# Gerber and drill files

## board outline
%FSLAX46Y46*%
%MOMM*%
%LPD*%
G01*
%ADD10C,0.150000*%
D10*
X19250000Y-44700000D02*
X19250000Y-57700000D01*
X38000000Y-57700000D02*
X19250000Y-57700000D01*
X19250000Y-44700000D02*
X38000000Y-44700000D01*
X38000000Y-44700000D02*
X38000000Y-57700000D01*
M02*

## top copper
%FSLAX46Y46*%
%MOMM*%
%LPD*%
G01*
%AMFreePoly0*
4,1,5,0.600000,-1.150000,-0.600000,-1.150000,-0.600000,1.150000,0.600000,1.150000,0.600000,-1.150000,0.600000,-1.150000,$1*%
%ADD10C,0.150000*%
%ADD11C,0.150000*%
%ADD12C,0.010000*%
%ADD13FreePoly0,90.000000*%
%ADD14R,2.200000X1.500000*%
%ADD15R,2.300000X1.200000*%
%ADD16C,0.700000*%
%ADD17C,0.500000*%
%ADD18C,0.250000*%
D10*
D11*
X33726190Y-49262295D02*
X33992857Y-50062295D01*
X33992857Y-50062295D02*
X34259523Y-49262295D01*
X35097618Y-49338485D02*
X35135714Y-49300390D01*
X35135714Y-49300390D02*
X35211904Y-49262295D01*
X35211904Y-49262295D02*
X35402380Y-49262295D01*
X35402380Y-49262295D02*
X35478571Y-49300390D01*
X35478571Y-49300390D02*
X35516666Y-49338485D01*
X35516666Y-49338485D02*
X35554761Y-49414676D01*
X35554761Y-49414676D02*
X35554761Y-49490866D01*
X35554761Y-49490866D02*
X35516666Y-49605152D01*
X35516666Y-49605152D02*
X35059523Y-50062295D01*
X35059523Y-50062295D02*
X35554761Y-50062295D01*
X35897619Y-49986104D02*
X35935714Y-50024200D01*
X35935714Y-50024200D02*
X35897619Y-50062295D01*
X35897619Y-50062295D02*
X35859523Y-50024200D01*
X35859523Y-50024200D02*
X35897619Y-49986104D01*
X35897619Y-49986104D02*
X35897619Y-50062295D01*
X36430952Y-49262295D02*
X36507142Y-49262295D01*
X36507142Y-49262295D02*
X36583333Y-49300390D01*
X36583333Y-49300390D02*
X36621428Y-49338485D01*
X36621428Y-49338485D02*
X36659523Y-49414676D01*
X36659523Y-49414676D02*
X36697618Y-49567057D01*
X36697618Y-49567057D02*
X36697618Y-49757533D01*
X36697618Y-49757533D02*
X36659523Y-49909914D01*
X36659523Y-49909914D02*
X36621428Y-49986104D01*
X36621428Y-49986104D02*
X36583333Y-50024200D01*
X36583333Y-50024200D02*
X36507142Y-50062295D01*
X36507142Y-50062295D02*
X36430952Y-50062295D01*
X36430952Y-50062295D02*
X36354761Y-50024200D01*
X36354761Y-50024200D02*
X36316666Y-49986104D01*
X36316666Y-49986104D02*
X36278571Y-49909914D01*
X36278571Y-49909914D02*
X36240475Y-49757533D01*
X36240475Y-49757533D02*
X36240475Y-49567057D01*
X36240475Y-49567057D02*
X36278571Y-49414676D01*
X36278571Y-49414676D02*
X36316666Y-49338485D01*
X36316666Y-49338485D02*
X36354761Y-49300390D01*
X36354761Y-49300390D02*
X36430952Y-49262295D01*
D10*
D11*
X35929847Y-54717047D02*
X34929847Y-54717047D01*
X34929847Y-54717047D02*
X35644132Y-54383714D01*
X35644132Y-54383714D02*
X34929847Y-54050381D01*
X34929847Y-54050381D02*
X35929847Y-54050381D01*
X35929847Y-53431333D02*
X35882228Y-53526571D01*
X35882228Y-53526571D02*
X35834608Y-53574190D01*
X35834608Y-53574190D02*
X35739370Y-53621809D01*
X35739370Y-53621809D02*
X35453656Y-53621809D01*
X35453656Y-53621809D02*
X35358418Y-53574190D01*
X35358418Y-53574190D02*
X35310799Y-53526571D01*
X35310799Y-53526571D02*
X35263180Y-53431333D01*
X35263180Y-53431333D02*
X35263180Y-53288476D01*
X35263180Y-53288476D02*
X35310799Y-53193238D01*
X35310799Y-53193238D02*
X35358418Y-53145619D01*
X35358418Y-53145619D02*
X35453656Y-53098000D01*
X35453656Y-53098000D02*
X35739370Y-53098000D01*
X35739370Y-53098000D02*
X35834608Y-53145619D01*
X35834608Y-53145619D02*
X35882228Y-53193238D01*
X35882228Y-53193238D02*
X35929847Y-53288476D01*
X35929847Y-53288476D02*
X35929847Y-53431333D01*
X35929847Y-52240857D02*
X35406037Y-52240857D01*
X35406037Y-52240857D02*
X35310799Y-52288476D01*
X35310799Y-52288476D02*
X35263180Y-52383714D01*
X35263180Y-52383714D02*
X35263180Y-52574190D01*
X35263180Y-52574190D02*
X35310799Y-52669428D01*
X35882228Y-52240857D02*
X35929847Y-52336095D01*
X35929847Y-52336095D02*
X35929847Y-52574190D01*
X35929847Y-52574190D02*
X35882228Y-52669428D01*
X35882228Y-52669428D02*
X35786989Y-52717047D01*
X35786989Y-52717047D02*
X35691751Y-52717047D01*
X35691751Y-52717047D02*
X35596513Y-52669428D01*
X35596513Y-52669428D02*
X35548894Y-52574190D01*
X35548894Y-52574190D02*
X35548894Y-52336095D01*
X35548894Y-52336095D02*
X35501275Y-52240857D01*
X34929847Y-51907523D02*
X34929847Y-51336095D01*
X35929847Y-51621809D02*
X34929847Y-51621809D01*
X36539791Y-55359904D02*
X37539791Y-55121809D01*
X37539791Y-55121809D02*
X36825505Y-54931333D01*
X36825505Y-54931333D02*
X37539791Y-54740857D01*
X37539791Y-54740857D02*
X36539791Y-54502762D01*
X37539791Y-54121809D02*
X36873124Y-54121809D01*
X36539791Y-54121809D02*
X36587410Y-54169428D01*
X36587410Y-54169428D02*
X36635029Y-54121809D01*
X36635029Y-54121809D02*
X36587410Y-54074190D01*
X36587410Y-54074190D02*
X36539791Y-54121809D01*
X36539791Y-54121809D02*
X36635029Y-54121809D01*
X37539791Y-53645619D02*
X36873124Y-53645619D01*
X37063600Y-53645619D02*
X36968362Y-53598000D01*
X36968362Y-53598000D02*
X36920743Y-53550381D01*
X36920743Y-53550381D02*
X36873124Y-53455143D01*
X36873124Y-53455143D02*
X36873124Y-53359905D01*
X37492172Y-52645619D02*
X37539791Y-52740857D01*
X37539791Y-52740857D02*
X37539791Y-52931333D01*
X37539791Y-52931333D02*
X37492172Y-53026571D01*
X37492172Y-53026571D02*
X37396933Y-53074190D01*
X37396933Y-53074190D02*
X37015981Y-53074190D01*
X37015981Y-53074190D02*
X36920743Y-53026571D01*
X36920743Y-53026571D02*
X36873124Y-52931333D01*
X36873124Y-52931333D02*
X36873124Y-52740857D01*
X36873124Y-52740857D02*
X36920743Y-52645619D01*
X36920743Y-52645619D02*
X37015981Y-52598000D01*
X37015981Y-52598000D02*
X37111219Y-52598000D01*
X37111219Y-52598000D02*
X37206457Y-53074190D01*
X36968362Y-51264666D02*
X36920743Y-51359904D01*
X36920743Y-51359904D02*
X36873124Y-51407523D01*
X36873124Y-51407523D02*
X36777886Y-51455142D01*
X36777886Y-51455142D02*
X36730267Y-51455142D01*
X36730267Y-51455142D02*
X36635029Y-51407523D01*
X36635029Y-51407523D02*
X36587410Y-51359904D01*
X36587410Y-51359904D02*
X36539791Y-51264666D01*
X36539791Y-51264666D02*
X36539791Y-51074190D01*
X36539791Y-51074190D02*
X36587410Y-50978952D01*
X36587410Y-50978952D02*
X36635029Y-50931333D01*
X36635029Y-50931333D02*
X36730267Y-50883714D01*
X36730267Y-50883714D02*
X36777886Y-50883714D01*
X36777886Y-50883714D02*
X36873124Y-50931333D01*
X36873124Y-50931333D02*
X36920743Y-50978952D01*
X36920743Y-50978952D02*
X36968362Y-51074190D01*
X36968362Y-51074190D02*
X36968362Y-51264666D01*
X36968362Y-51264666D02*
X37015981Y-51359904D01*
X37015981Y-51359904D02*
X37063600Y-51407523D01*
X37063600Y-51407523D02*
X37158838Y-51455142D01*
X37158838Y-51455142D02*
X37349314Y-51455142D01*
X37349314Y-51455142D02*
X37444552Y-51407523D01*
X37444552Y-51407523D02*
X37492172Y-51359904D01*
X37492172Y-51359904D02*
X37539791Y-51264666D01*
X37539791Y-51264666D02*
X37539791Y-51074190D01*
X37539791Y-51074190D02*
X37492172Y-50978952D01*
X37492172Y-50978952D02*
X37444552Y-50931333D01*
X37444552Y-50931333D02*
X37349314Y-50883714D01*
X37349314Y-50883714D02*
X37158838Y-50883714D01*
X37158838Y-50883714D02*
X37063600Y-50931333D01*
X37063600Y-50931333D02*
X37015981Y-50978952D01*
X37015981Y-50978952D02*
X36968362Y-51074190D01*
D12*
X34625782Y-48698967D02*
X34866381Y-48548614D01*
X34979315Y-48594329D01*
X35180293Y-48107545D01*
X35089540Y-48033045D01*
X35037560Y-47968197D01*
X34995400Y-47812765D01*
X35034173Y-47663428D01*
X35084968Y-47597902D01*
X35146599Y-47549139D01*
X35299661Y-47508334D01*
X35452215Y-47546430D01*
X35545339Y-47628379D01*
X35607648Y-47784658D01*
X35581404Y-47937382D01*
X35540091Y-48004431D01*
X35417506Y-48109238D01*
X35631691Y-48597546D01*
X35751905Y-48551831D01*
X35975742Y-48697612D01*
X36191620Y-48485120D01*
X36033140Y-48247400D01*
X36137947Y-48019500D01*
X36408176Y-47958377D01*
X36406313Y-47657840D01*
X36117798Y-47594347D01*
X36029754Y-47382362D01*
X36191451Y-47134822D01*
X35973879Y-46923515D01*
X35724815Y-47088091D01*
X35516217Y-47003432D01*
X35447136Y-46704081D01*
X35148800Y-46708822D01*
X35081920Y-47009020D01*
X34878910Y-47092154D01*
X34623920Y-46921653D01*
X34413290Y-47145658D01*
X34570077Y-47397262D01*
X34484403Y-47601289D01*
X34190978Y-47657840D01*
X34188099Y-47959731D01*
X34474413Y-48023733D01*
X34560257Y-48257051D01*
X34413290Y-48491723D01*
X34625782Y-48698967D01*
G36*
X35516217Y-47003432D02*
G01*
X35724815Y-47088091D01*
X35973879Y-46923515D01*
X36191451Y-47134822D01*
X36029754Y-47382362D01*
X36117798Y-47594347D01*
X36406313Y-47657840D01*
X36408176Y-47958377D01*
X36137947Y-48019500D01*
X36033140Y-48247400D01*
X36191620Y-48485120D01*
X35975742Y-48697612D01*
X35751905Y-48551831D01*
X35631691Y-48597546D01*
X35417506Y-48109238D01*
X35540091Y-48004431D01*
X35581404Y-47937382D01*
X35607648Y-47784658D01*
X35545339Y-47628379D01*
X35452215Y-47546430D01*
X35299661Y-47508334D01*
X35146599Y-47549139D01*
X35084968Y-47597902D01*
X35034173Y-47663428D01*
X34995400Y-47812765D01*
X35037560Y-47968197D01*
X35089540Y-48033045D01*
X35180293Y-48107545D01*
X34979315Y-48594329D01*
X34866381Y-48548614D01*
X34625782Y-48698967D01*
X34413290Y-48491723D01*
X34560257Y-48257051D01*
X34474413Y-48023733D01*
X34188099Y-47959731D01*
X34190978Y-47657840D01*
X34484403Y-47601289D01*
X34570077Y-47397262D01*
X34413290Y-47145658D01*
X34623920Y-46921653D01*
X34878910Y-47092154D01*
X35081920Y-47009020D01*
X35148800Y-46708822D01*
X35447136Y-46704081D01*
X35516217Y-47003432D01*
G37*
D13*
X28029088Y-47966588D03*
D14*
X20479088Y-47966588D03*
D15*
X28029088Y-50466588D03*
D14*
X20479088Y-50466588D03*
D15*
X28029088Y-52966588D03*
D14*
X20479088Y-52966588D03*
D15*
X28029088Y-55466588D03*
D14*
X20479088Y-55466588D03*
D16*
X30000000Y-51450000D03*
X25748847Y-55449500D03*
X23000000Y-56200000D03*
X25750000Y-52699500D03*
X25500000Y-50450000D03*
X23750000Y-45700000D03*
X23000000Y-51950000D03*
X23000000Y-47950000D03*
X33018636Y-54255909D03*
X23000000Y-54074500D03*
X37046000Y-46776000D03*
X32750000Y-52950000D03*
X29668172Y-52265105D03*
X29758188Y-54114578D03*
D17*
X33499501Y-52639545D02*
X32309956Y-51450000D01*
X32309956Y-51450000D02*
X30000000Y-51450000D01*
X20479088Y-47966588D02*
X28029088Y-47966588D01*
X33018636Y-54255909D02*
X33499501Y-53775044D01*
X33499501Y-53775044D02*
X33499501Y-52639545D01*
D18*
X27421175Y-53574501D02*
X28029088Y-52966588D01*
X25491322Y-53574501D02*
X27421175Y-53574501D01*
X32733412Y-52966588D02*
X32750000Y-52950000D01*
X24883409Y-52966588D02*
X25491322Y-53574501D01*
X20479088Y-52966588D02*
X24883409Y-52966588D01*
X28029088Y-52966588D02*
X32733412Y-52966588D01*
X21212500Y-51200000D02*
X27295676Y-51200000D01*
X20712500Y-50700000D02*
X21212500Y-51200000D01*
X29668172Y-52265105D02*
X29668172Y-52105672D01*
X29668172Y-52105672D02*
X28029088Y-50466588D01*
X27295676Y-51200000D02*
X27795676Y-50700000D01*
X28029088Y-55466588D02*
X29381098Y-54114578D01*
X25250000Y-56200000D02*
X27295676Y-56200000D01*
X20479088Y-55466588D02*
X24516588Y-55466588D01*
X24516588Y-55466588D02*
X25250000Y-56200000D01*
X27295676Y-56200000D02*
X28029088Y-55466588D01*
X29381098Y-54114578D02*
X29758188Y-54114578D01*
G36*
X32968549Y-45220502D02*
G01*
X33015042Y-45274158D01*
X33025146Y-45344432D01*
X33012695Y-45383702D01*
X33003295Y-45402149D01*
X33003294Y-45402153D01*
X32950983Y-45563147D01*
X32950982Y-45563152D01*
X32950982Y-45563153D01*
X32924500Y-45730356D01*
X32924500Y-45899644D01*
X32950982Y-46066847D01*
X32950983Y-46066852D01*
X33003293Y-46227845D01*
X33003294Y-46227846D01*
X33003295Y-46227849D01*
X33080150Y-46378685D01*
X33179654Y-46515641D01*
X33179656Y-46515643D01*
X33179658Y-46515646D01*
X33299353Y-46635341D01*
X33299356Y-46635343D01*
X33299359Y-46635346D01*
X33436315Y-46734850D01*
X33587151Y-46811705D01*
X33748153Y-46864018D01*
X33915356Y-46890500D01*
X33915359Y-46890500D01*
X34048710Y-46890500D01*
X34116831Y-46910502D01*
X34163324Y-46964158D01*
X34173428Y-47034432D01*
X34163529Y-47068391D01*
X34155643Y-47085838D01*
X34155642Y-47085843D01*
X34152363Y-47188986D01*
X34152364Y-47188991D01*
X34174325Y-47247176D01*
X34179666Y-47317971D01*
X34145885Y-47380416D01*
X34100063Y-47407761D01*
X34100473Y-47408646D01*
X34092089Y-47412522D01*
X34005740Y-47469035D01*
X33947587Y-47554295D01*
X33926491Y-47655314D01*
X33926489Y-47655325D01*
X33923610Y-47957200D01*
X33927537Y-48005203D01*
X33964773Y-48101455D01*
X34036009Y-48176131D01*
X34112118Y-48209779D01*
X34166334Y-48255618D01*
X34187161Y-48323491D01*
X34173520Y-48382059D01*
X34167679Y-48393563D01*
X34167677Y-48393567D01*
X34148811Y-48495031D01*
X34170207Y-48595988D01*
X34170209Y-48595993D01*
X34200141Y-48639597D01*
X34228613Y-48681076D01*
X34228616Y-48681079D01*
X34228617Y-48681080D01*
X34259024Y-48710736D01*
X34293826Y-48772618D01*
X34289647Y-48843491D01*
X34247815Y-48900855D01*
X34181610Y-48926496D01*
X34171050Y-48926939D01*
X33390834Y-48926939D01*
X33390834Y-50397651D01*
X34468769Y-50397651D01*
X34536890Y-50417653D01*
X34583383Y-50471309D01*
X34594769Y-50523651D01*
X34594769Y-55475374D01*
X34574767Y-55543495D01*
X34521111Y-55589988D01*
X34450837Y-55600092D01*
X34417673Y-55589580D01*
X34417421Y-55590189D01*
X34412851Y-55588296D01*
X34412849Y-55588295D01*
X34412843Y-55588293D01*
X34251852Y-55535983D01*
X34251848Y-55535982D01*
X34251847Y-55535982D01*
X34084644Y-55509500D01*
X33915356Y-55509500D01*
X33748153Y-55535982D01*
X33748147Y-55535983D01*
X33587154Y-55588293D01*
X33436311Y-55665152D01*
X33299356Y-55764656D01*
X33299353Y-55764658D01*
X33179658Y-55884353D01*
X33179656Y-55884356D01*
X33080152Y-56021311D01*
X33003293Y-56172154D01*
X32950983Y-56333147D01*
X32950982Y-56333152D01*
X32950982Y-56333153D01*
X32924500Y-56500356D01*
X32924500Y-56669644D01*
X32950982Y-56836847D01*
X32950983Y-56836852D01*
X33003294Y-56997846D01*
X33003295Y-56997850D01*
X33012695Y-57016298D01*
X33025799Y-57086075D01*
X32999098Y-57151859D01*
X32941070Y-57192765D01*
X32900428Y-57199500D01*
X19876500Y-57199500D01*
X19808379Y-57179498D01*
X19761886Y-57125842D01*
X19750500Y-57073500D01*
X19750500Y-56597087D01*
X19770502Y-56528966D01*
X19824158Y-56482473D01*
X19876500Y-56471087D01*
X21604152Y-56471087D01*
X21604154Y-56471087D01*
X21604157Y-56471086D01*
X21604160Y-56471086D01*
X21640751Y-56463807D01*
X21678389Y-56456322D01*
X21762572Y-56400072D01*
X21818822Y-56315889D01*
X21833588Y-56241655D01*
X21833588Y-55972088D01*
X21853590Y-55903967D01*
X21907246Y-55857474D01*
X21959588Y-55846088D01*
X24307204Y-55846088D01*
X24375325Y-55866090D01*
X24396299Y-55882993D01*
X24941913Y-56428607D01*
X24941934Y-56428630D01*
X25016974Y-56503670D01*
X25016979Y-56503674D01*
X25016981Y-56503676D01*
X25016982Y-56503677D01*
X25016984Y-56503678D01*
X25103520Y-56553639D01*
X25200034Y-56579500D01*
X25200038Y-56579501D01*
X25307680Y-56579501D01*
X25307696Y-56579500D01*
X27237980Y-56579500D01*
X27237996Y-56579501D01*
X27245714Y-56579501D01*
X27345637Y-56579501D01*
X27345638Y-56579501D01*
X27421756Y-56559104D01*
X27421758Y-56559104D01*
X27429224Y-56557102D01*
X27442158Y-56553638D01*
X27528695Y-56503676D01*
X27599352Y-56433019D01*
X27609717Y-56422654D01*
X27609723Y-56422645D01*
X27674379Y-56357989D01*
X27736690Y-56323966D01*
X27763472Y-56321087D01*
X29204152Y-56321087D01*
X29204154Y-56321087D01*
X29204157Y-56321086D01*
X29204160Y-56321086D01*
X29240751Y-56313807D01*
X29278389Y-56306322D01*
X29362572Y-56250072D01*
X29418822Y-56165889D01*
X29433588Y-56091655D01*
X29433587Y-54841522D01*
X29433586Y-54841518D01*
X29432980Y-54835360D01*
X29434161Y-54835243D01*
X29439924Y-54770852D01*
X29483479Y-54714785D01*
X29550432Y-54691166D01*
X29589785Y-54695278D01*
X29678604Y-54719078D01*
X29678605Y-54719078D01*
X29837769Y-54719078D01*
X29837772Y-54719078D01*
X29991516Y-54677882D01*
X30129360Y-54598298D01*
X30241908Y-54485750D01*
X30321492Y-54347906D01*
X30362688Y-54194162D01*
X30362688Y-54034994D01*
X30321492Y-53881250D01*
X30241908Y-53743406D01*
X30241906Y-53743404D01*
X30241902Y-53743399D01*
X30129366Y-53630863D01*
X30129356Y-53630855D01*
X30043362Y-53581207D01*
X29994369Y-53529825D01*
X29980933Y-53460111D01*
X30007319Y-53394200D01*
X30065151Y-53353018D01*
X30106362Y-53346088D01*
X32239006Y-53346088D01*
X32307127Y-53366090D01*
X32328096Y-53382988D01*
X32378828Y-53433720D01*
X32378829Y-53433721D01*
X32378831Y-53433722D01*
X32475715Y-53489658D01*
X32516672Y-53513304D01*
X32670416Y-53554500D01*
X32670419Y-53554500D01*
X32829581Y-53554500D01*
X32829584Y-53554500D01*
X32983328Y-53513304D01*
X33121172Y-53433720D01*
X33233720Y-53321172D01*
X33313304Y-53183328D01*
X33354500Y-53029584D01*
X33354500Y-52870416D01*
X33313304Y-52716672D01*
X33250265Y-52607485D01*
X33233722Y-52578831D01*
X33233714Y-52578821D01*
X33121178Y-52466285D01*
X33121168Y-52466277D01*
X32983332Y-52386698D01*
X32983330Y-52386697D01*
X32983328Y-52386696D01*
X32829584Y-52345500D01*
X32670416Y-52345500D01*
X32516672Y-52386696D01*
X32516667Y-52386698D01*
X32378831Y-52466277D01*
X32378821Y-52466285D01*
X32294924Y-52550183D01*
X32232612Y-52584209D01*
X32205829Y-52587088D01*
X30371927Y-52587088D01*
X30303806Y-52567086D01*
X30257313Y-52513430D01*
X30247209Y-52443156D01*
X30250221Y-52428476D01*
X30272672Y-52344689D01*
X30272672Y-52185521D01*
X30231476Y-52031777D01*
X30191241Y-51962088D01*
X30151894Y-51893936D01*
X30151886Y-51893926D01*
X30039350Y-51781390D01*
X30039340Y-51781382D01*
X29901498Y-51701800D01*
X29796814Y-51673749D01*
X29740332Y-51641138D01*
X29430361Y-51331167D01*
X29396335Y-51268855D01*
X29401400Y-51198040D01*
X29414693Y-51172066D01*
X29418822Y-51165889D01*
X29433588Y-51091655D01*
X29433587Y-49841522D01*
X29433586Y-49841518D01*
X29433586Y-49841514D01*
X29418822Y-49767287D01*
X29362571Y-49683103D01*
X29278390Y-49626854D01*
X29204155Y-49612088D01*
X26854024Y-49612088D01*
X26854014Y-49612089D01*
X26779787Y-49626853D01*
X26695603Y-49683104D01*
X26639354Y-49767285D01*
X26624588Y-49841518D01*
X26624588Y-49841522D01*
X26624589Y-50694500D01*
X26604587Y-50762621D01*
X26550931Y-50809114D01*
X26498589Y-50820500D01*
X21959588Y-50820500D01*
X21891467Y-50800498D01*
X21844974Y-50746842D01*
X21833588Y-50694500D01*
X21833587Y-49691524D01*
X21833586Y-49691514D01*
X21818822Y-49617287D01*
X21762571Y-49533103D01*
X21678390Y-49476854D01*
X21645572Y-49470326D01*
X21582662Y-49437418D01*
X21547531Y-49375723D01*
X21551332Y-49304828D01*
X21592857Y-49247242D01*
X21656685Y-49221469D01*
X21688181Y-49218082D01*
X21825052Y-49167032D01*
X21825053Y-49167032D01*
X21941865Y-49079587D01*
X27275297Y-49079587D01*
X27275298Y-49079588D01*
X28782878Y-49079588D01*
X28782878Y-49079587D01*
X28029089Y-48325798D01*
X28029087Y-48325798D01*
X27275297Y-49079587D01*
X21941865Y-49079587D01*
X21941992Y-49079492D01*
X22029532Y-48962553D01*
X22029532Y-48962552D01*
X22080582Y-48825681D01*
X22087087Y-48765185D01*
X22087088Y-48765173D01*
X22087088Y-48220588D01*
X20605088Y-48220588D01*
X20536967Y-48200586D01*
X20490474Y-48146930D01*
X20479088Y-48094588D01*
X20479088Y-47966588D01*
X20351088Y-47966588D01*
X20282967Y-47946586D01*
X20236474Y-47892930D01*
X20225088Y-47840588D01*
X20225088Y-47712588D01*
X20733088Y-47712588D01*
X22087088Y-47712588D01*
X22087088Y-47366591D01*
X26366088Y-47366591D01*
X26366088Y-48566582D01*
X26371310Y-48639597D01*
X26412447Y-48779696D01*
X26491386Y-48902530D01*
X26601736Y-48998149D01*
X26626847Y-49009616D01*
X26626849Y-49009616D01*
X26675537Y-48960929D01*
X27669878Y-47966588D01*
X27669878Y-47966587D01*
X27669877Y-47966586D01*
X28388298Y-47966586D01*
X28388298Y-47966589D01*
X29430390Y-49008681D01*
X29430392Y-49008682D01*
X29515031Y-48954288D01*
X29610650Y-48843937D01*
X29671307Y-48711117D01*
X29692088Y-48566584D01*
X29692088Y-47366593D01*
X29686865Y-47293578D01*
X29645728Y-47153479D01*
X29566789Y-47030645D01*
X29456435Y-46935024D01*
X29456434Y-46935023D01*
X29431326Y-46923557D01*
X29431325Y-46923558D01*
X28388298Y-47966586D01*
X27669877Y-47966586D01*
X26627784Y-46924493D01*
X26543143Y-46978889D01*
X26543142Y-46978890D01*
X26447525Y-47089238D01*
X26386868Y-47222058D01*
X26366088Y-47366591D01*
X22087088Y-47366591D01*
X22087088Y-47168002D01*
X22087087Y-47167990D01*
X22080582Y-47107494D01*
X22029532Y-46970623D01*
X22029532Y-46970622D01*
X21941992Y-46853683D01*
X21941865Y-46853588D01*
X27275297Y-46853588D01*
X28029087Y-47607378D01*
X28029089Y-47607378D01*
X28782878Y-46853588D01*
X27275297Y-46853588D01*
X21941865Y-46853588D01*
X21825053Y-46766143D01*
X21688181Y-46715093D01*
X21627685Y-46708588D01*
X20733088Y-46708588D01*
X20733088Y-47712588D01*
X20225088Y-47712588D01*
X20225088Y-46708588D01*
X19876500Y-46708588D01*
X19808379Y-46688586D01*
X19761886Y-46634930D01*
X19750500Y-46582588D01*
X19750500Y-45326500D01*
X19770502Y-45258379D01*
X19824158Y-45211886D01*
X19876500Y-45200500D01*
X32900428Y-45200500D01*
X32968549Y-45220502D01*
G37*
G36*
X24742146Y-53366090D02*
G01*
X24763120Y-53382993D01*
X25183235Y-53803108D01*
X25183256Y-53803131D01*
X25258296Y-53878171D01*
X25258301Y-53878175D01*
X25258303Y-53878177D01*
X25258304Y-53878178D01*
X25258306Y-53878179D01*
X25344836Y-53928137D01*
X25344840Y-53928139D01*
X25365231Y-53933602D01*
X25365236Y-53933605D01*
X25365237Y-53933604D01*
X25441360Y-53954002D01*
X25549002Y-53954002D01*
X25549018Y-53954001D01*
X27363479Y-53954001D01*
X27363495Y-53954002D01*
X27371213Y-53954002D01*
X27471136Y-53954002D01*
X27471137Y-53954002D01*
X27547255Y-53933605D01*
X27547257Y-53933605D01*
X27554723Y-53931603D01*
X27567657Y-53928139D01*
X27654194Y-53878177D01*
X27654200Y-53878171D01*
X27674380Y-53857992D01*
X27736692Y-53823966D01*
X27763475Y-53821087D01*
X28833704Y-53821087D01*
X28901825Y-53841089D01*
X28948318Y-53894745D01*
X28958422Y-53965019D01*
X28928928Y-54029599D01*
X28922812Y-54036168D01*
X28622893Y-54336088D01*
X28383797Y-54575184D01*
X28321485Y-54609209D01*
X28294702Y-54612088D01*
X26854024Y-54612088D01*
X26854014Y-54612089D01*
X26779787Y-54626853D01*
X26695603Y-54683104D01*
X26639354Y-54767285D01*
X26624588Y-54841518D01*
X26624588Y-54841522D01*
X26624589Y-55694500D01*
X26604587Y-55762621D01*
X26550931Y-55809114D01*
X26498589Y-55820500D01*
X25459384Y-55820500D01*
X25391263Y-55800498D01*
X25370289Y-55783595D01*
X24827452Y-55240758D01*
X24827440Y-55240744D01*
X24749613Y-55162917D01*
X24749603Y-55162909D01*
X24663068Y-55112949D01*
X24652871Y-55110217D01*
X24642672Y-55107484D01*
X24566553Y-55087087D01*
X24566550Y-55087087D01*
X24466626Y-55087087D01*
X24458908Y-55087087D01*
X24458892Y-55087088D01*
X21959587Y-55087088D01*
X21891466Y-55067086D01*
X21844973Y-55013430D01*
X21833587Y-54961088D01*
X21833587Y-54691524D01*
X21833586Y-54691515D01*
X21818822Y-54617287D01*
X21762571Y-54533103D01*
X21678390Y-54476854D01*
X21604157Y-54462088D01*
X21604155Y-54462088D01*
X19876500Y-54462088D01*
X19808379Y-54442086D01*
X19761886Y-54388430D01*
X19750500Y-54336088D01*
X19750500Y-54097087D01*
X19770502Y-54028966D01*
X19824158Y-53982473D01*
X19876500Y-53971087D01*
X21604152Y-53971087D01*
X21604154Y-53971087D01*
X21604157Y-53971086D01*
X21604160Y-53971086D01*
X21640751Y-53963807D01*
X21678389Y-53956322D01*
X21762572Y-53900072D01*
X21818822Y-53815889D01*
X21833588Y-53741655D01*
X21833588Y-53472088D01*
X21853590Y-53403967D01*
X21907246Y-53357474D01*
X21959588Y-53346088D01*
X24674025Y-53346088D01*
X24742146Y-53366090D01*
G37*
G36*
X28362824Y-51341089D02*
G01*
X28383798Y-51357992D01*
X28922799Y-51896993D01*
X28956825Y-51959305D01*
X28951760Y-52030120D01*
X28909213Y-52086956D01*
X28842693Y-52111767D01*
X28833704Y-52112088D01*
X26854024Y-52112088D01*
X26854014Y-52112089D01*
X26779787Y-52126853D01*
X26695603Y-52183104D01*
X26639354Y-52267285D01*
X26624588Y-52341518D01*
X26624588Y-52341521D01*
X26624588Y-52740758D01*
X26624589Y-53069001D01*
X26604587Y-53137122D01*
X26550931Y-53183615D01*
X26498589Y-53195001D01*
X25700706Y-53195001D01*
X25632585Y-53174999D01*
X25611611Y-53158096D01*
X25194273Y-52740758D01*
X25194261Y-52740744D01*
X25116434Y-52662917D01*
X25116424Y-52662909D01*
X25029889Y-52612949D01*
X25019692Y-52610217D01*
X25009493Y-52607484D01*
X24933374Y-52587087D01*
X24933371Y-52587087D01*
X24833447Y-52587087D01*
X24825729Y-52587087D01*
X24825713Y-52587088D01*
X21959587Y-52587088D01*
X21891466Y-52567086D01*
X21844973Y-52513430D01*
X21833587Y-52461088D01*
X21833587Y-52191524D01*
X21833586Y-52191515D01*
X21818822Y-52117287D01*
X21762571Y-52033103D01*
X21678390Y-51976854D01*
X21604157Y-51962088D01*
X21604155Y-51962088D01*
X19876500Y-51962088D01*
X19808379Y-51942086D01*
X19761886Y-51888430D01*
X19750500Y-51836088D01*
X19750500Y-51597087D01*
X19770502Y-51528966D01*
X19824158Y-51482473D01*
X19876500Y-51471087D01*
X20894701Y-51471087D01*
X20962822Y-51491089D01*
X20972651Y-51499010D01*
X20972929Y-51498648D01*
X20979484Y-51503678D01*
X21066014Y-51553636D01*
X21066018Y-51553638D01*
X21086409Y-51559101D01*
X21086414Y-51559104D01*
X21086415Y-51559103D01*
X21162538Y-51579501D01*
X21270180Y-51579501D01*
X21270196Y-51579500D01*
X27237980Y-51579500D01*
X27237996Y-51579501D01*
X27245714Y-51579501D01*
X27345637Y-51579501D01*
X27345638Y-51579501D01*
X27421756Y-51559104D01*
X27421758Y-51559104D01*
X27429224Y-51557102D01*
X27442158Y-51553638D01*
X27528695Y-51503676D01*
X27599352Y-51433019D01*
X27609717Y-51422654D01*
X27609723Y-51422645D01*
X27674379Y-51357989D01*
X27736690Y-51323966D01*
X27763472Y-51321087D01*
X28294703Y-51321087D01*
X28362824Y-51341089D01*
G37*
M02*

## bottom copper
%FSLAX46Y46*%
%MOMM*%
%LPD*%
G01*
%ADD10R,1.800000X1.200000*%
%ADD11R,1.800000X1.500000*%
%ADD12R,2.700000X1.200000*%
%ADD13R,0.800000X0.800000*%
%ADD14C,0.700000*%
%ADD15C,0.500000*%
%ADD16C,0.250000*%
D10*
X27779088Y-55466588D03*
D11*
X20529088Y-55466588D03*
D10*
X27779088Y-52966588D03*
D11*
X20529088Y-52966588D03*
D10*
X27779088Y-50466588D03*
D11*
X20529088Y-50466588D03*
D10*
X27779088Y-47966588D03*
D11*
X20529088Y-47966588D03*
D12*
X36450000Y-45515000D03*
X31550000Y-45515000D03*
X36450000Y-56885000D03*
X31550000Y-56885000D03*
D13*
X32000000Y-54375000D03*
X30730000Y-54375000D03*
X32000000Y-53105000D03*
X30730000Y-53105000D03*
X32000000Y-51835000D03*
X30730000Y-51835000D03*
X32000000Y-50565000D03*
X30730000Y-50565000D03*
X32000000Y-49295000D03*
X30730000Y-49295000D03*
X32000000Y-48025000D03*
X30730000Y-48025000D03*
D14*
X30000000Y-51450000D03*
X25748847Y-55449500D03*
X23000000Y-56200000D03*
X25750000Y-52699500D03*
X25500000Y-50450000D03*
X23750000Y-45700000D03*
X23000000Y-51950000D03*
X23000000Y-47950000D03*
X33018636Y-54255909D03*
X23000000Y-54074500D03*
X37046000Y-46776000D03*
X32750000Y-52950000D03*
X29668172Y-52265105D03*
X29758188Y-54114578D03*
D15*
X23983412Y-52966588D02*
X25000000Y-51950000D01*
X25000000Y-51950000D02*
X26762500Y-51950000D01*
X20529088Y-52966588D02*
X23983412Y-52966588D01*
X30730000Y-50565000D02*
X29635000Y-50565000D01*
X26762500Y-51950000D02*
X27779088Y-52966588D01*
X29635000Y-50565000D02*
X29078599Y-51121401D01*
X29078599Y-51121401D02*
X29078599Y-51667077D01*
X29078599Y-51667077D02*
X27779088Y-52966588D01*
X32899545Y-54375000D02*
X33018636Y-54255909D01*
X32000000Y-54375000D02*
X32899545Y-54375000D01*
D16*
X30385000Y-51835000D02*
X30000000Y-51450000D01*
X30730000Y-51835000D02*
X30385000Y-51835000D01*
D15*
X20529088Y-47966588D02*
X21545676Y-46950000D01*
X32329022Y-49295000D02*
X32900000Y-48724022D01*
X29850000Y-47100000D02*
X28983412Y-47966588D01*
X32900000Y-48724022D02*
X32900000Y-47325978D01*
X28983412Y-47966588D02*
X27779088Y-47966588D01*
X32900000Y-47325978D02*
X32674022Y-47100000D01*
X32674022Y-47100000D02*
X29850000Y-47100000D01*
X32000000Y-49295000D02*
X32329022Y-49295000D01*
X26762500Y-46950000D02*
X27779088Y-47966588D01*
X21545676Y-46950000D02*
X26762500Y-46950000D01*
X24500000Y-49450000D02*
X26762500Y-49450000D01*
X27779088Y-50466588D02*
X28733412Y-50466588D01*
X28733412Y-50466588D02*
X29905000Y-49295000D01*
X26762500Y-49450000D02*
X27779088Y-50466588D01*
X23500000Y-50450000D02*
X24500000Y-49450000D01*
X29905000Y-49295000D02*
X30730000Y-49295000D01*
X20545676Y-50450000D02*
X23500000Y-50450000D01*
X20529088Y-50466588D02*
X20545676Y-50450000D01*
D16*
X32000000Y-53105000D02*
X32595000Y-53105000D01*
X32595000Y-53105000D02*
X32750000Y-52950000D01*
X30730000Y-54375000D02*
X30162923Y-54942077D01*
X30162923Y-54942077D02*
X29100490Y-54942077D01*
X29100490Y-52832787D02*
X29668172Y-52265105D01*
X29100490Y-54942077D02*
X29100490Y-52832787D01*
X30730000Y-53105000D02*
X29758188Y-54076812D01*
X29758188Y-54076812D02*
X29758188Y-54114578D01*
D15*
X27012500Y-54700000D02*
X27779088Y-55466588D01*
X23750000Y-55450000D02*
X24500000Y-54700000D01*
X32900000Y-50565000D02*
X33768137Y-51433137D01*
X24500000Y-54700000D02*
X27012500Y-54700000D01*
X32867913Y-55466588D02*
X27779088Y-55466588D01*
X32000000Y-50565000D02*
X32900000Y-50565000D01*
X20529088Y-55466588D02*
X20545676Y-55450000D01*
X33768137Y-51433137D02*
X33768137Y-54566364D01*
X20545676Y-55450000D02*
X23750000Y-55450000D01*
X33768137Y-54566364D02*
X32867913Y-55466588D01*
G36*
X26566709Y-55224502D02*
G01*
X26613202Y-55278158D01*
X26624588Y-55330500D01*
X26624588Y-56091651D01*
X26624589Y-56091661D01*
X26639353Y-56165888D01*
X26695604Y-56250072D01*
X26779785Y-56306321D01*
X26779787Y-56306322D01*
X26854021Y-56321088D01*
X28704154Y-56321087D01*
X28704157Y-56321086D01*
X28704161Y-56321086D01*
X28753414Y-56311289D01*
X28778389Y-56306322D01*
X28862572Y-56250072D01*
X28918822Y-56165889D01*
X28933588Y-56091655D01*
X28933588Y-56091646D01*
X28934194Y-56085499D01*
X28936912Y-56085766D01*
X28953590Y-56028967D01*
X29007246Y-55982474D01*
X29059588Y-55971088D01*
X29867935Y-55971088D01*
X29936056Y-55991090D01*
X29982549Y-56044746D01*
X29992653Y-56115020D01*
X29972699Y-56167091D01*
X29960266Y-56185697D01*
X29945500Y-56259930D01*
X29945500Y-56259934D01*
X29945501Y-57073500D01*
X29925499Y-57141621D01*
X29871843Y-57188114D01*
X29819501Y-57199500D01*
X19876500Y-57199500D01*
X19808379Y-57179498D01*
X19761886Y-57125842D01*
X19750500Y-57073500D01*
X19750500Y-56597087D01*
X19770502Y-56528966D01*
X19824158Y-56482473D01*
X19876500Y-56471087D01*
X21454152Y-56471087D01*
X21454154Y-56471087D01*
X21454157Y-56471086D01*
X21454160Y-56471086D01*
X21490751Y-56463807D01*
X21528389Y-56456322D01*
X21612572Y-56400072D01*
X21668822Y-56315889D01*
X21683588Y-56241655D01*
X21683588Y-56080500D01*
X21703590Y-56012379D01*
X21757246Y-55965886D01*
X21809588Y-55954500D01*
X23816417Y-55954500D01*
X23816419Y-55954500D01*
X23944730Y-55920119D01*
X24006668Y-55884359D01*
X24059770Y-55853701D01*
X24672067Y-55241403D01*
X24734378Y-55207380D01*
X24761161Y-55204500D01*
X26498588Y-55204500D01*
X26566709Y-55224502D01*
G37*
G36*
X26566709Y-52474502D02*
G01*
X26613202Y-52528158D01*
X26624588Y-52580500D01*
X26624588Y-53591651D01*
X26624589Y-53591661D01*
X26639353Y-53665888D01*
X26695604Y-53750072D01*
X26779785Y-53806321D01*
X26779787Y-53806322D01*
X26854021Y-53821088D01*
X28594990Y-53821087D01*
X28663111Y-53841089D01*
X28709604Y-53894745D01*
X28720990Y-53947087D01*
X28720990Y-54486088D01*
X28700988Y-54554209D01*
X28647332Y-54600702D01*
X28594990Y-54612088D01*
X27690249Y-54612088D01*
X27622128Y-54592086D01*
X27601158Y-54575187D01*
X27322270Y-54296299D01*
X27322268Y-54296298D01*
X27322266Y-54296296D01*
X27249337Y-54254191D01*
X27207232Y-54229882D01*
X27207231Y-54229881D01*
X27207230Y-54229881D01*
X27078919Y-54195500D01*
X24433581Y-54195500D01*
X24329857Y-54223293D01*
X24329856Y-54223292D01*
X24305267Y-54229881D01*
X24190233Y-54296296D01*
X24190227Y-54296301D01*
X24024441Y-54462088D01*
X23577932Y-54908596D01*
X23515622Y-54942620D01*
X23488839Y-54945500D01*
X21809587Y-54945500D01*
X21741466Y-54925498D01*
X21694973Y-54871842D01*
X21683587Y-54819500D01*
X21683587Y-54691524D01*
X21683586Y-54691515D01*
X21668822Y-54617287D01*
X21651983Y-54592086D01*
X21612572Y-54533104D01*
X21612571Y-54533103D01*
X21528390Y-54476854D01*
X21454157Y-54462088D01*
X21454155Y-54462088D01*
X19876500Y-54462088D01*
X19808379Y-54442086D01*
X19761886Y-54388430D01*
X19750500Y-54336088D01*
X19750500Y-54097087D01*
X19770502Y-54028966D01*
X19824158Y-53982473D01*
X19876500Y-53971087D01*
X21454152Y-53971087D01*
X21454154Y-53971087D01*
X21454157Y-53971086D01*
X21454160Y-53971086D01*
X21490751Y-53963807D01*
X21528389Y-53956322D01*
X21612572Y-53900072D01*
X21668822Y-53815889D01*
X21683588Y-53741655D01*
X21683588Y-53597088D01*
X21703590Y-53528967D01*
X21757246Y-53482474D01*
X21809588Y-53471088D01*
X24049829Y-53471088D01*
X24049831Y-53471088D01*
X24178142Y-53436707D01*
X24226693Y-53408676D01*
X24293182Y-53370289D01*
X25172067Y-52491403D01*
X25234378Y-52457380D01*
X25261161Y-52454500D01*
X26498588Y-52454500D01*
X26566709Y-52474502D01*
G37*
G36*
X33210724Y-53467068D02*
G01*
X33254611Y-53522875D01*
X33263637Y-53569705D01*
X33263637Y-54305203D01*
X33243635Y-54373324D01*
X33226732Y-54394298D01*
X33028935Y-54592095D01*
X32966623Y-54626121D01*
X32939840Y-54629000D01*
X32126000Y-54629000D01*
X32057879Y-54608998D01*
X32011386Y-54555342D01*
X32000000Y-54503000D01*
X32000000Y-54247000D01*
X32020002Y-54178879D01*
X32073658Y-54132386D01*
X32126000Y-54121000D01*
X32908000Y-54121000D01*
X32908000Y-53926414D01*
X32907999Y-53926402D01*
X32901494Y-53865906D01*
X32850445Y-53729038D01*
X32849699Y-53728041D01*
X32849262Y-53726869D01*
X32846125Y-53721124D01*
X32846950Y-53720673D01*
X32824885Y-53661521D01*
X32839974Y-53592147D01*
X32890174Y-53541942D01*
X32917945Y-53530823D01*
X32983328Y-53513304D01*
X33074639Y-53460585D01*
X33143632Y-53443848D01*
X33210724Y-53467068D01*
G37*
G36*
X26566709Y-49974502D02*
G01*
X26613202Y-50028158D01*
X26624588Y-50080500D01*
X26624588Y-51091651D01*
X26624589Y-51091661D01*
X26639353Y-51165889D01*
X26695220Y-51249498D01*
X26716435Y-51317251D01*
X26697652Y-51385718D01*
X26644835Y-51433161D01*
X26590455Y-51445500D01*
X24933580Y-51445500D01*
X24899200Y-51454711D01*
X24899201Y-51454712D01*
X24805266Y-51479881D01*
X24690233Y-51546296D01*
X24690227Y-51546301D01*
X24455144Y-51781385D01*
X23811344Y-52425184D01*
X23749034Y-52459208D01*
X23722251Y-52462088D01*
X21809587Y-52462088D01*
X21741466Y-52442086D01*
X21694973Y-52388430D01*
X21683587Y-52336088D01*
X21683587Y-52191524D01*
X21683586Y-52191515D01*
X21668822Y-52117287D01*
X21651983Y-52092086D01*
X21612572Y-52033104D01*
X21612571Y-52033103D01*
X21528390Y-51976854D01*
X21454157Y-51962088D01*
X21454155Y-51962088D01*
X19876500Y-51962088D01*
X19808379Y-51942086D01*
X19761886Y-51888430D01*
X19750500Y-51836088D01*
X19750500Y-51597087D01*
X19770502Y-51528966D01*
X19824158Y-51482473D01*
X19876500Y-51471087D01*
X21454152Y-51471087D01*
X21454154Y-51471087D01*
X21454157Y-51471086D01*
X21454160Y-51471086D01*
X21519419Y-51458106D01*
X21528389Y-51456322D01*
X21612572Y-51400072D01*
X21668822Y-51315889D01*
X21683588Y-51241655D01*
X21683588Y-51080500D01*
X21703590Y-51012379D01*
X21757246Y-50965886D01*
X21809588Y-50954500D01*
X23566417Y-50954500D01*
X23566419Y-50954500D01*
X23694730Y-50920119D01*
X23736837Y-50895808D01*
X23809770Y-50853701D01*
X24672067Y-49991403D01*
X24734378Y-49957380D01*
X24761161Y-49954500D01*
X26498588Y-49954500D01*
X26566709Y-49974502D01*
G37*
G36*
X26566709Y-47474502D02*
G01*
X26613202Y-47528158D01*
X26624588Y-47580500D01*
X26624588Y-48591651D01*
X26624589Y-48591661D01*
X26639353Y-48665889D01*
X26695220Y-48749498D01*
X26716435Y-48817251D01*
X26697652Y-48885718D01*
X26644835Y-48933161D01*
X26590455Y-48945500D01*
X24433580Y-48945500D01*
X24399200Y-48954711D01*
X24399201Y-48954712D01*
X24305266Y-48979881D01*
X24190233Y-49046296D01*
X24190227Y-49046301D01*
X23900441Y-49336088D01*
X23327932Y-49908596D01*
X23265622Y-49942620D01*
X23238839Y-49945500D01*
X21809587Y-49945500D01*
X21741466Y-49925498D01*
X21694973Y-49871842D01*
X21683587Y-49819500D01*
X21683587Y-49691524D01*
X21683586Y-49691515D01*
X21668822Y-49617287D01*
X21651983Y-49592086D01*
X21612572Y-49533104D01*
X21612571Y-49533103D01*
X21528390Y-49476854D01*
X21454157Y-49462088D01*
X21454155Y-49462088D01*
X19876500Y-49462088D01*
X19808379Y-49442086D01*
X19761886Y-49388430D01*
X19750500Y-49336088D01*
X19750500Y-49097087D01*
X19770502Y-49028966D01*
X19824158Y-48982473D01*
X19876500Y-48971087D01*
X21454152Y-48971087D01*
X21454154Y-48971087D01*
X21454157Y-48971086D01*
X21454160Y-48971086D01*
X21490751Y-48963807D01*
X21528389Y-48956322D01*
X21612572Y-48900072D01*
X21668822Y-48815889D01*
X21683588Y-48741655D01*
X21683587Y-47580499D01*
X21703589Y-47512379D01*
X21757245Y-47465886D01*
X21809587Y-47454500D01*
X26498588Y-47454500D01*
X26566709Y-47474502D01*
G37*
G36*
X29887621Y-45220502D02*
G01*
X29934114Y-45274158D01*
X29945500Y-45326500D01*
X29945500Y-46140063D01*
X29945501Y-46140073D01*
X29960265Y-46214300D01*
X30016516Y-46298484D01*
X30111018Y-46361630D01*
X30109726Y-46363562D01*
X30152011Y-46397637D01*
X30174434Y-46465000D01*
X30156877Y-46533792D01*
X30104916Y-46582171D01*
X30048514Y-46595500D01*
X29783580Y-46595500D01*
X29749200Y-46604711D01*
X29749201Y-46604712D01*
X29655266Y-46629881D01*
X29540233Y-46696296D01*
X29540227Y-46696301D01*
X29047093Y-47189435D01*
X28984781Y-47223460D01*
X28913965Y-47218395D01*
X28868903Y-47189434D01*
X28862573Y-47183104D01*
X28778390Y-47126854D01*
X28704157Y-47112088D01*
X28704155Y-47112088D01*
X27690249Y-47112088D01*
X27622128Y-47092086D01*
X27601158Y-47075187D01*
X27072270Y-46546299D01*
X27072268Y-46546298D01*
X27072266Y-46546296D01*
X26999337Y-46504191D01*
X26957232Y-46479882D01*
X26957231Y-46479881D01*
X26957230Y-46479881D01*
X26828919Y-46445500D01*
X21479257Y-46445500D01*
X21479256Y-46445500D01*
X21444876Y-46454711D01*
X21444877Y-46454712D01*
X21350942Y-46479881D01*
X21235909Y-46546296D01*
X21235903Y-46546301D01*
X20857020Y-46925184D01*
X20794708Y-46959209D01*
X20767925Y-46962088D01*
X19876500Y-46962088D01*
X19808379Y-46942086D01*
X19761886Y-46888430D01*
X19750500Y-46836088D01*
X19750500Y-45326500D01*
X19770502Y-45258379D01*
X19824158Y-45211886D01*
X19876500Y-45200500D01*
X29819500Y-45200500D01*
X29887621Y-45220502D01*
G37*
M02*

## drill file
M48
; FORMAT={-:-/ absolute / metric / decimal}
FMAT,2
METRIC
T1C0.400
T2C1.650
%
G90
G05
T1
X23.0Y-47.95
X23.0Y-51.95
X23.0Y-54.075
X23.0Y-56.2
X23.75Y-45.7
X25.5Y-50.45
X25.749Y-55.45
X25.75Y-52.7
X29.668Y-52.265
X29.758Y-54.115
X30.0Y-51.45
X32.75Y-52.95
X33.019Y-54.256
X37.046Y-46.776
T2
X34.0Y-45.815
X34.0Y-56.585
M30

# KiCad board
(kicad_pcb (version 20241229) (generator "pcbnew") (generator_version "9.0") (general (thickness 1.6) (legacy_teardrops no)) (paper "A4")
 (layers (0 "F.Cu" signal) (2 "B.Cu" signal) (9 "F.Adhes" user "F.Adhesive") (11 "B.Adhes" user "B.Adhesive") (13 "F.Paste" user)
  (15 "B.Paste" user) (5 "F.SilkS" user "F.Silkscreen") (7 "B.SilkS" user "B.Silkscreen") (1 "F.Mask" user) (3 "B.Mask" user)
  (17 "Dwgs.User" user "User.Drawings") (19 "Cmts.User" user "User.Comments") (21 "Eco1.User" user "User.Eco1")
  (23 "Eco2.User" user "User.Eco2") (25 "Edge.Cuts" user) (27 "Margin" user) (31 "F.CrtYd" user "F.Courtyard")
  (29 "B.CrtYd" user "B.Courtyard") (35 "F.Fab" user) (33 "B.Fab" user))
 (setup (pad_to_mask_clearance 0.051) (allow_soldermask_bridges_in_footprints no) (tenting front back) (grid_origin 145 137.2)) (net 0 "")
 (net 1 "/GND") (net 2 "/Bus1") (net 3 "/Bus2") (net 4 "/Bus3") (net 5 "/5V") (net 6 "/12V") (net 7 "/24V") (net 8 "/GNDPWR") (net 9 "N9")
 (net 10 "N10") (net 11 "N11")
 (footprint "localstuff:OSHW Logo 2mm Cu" (layer "F.Cu") (at 35.3 47.7)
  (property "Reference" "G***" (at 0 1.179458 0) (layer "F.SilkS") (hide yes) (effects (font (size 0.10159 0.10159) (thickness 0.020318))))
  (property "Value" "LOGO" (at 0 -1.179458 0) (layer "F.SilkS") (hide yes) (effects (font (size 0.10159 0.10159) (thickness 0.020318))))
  (fp_poly
   (pts (xy -0.674218 0.998967) (xy -0.433619 0.848614) (xy -0.320685 0.894329) (xy -0.119707 0.407545) (xy -0.21046 0.333045)
    (xy -0.26244 0.268197) (xy -0.3046 0.112765) (xy -0.265827 -0.036572) (xy -0.215032 -0.102098) (xy -0.153401 -0.150861)
    (xy -0.000339 -0.191666) (xy 0.152215 -0.15357) (xy 0.245339 -0.071621) (xy 0.307648 0.084658) (xy 0.281404 0.237382)
    (xy 0.240091 0.304431) (xy 0.117506 0.409238) (xy 0.331691 0.897546) (xy 0.451905 0.851831) (xy 0.675742 0.997612) (xy 0.89162 0.78512)
    (xy 0.73314 0.5474) (xy 0.837947 0.3195) (xy 1.108176 0.258377) (xy 1.106313 -0.04216) (xy 0.817798 -0.105653) (xy 0.729754 -0.317638)
    (xy 0.891451 -0.565178) (xy 0.673879 -0.776485) (xy 0.424815 -0.611909) (xy 0.216217 -0.696568) (xy 0.147136 -0.995919)
    (xy -0.1512 -0.991178) (xy -0.21808 -0.69098) (xy -0.42109 -0.607846) (xy -0.67608 -0.778347) (xy -0.88671 -0.554342)
    (xy -0.729923 -0.302738) (xy -0.815597 -0.098711) (xy -1.109022 -0.04216) (xy -1.111901 0.259731) (xy -0.825587 0.323733)
    (xy -0.739743 0.557051) (xy -0.88671 0.791723) (xy -0.674218 0.998967))
   (stroke (width 0.01) (type solid)) (fill yes) (layer "F.Cu")))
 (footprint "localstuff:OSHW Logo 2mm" (layer "F.Cu") (at 35.3 47.7)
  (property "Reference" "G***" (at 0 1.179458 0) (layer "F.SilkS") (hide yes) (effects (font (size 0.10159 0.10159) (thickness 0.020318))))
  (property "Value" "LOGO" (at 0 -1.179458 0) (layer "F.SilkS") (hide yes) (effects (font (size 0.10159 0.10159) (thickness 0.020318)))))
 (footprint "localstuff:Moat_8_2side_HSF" (layer "F.Cu") (at 24.279088 56.716588 -90)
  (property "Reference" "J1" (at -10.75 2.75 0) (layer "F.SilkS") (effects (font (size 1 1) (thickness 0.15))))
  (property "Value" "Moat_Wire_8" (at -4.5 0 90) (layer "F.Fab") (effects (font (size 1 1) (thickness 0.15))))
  (pad "1" smd custom (at -8.75 -3.75 90) (size 1.2 2.3) (layers "F.Cu" "F.Mask" "F.Paste") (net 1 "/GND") (thermal_bridge_angle 45)
   (options (clearance outline) (anchor rect)) (primitives))
  (pad "1" smd rect (at -8.75 3.8 270) (size 1.5 2.2) (layers "F.Cu" "F.Mask" "F.Paste") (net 1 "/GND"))
  (pad "2" smd rect (at -6.25 -3.75 270) (size 1.2 2.3) (layers "F.Cu" "F.Mask" "F.Paste") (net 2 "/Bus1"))
  (pad "2" smd rect (at -6.25 3.8 270) (size 1.5 2.2) (layers "F.Cu" "F.Mask" "F.Paste") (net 2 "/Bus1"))
  (pad "3" smd rect (at -3.75 -3.75 270) (size 1.2 2.3) (layers "F.Cu" "F.Mask" "F.Paste") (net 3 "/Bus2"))
  (pad "3" smd rect (at -3.75 3.8 270) (size 1.5 2.2) (layers "F.Cu" "F.Mask" "F.Paste") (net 3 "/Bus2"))
  (pad "4" smd rect (at -1.25 -3.75 270) (size 1.2 2.3) (layers "F.Cu" "F.Mask" "F.Paste") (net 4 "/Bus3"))
  (pad "4" smd rect (at -1.25 3.8 270) (size 1.5 2.2) (layers "F.Cu" "F.Mask" "F.Paste") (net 4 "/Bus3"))
  (pad "5" smd rect (at -1.25 -3.5 90) (size 1.2 1.8) (layers "B.Cu" "B.Mask" "B.Paste") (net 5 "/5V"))
  (pad "5" smd rect (at -1.25 3.75 90) (size 1.5 1.8) (layers "B.Cu" "B.Mask" "B.Paste") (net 5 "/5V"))
  (pad "6" smd rect (at -3.75 -3.5 90) (size 1.2 1.8) (layers "B.Cu" "B.Mask" "B.Paste") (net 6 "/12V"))
  (pad "6" smd rect (at -3.75 3.75 90) (size 1.5 1.8) (layers "B.Cu" "B.Mask" "B.Paste") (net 6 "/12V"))
  (pad "7" smd rect (at -6.25 -3.5 90) (size 1.2 1.8) (layers "B.Cu" "B.Mask" "B.Paste") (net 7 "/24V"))
  (pad "7" smd rect (at -6.25 3.75 90) (size 1.5 1.8) (layers "B.Cu" "B.Mask" "B.Paste") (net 7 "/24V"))
  (pad "8" smd rect (at -8.75 -3.5 90) (size 1.2 1.8) (layers "B.Cu" "B.Mask" "B.Paste") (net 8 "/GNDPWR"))
  (pad "8" smd rect (at -8.75 3.75 90) (size 1.5 1.8) (layers "B.Cu" "B.Mask" "B.Paste") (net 8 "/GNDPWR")))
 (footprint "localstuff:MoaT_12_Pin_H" (layer "B.Cu") (at 34 51.2 -90)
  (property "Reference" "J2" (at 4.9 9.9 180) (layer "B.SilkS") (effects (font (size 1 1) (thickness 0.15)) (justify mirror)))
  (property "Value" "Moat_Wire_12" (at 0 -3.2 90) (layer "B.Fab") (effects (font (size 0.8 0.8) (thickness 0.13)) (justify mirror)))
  (pad "" smd rect (at -5.685 -2.45 180) (size 2.7 1.2) (layers "B.Cu" "B.Mask" "B.Paste"))
  (pad "" smd rect (at -5.685 2.45 180) (size 2.7 1.2) (layers "B.Cu" "B.Mask" "B.Paste"))
  (pad "" np_thru_hole circle (at -5.385 0 180) (size 1.65 1.65) (drill 1.65) (layers "*.Cu"))
  (pad "" np_thru_hole circle (at 5.385 0) (size 1.65 1.65) (drill 1.65) (layers "*.Cu"))
  (pad "" smd rect (at 5.685 -2.45) (size 2.7 1.2) (layers "B.Cu" "B.Mask" "B.Paste"))
  (pad "" smd rect (at 5.685 2.45) (size 2.7 1.2) (layers "B.Cu" "B.Mask" "B.Paste"))
  (pad "1" smd rect (at 3.175 2) (size 0.8 0.8) (layers "B.Cu" "B.Mask" "B.Paste") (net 1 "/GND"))
  (pad "2" smd rect (at 3.175 3.27) (size 0.8 0.8) (layers "B.Cu" "B.Mask" "B.Paste") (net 2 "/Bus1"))
  (pad "3" smd rect (at 1.905 2) (size 0.8 0.8) (layers "B.Cu" "B.Mask" "B.Paste") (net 3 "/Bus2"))
  (pad "4" smd rect (at 1.905 3.27) (size 0.8 0.8) (layers "B.Cu" "B.Mask" "B.Paste") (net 4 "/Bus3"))
  (pad "5" smd rect (at 0.635 2) (size 0.8 0.8) (layers "B.Cu" "B.Mask" "B.Paste") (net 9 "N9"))
  (pad "6" smd rect (at 0.635 3.27) (size 0.8 0.8) (layers "B.Cu" "B.Mask" "B.Paste") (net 1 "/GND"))
  (pad "7" smd rect (at -0.635 2) (size 0.8 0.8) (layers "B.Cu" "B.Mask" "B.Paste") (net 5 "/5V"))
  (pad "8" smd rect (at -0.635 3.27) (size 0.8 0.8) (layers "B.Cu" "B.Mask" "B.Paste") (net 6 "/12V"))
  (pad "9" smd rect (at -1.905 2) (size 0.8 0.8) (layers "B.Cu" "B.Mask" "B.Paste") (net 8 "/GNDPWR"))
  (pad "10" smd rect (at -1.905 3.27) (size 0.8 0.8) (layers "B.Cu" "B.Mask" "B.Paste") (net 7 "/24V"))
  (pad "11" smd rect (at -3.175 2) (size 0.8 0.8) (layers "B.Cu" "B.Mask" "B.Paste") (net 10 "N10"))
  (pad "12" smd rect (at -3.175 3.27) (size 0.8 0.8) (layers "B.Cu" "B.Mask" "B.Paste") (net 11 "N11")))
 (gr_line (start 19.25 44.7) (end 19.25 57.7) (stroke (width 0.15) (type solid)) (layer "Edge.Cuts"))
 (gr_line (start 38 57.7) (end 19.25 57.7) (stroke (width 0.15) (type solid)) (layer "Edge.Cuts"))
 (gr_line (start 19.25 44.7) (end 38 44.7) (stroke (width 0.15) (type solid)) (layer "Edge.Cuts"))
 (gr_line (start 38 44.7) (end 38 57.7) (stroke (width 0.15) (type solid)) (layer "Edge.Cuts"))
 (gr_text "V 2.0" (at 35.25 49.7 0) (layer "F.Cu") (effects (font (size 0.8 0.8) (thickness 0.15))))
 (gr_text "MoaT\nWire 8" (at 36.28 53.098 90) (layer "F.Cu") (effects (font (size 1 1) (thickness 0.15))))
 (segment (start 23.983412 52.966588) (end 25 51.95) (width 0.5) (layer "B.Cu") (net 6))
 (segment (start 25 51.95) (end 26.7625 51.95) (width 0.5) (layer "B.Cu") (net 6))
 (segment (start 20.529088 52.966588) (end 23.983412 52.966588) (width 0.5) (layer "B.Cu") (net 6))
 (segment (start 30.73 50.565) (end 29.635 50.565) (width 0.5) (layer "B.Cu") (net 6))
 (segment (start 26.7625 51.95) (end 27.779088 52.966588) (width 0.5) (layer "B.Cu") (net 6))
 (segment (start 29.635 50.565) (end 29.078599 51.121401) (width 0.5) (layer "B.Cu") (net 6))
 (segment (start 29.078599 51.121401) (end 29.078599 51.667077) (width 0.5) (layer "B.Cu") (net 6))
 (segment (start 29.078599 51.667077) (end 27.779088 52.966588) (width 0.5) (layer "B.Cu") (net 6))
 (segment (start 33.499501 52.639545) (end 32.309956 51.45) (width 0.5) (layer "F.Cu") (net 1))
 (segment (start 32.309956 51.45) (end 30 51.45) (width 0.5) (layer "F.Cu") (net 1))
 (segment (start 20.479088 47.966588) (end 28.029088 47.966588) (width 0.5) (layer "F.Cu") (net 1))
 (segment (start 33.018636 54.255909) (end 33.499501 53.775044) (width 0.5) (layer "F.Cu") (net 1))
 (segment (start 33.499501 53.775044) (end 33.499501 52.639545) (width 0.5) (layer "F.Cu") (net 1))
 (via (at 30 51.45) (size 0.7) (drill 0.4) (layers "F.Cu" "B.Cu") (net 1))
 (via (at 25.748847 55.4495) (size 0.7) (drill 0.4) (layers "F.Cu" "B.Cu") (free yes) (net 1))
 (via (at 23 56.2) (size 0.7) (drill 0.4) (layers "F.Cu" "B.Cu") (free yes) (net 1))
 (via (at 25.75 52.6995) (size 0.7) (drill 0.4) (layers "F.Cu" "B.Cu") (free yes) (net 1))
 (via (at 25.5 50.45) (size 0.7) (drill 0.4) (layers "F.Cu" "B.Cu") (free yes) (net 1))
 (via (at 23.75 45.7) (size 0.7) (drill 0.4) (layers "F.Cu" "B.Cu") (free yes) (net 1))
 (via (at 23 51.95) (size 0.7) (drill 0.4) (layers "F.Cu" "B.Cu") (free yes) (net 1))
 (via (at 23 47.95) (size 0.7) (drill 0.4) (layers "F.Cu" "B.Cu") (free yes) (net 1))
 (via (at 33.018636 54.255909) (size 0.7) (drill 0.4) (layers "F.Cu" "B.Cu") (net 1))
 (via (at 23 54.0745) (size 0.7) (drill 0.4) (layers "F.Cu" "B.Cu") (free yes) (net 1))
 (via (at 37.046 46.776) (size 0.7) (drill 0.4) (layers "F.Cu" "B.Cu") (free yes) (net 1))
 (segment (start 32.899545 54.375) (end 33.018636 54.255909) (width 0.5) (layer "B.Cu") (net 1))
 (segment (start 32 54.375) (end 32.899545 54.375) (width 0.5) (layer "B.Cu") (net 1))
 (segment (start 30.385 51.835) (end 30 51.45) (width 0.25) (layer "B.Cu") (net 1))
 (segment (start 30.73 51.835) (end 30.385 51.835) (width 0.25) (layer "B.Cu") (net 1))
 (segment (start 20.529088 47.966588) (end 21.545676 46.95) (width 0.5) (layer "B.Cu") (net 8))
 (segment (start 32.329022 49.295) (end 32.9 48.724022) (width 0.5) (layer "B.Cu") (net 8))
 (segment (start 29.85 47.1) (end 28.983412 47.966588) (width 0.5) (layer "B.Cu") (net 8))
 (segment (start 32.9 48.724022) (end 32.9 47.325978) (width 0.5) (layer "B.Cu") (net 8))
 (segment (start 28.983412 47.966588) (end 27.779088 47.966588) (width 0.5) (layer "B.Cu") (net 8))
 (segment (start 32.9 47.325978) (end 32.674022 47.1) (width 0.5) (layer "B.Cu") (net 8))
 (segment (start 32.674022 47.1) (end 29.85 47.1) (width 0.5) (layer "B.Cu") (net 8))
 (segment (start 32 49.295) (end 32.329022 49.295) (width 0.5) (layer "B.Cu") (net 8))
 (segment (start 26.7625 46.95) (end 27.779088 47.966588) (width 0.5) (layer "B.Cu") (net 8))
 (segment (start 21.545676 46.95) (end 26.7625 46.95) (width 0.5) (layer "B.Cu") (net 8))
 (segment (start 24.5 49.45) (end 26.7625 49.45) (width 0.5) (layer "B.Cu") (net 7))
 (segment (start 27.779088 50.466588) (end 28.733412 50.466588) (width 0.5) (layer "B.Cu") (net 7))
 (segment (start 28.733412 50.466588) (end 29.905 49.295) (width 0.5) (layer "B.Cu") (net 7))
 (segment (start 26.7625 49.45) (end 27.779088 50.466588) (width 0.5) (layer "B.Cu") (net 7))
 (segment (start 23.5 50.45) (end 24.5 49.45) (width 0.5) (layer "B.Cu") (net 7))
 (segment (start 29.905 49.295) (end 30.73 49.295) (width 0.5) (layer "B.Cu") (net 7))
 (segment (start 20.545676 50.45) (end 23.5 50.45) (width 0.5) (layer "B.Cu") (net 7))
 (segment (start 20.529088 50.466588) (end 20.545676 50.45) (width 0.5) (layer "B.Cu") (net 7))
 (segment (start 27.421175 53.574501) (end 28.029088 52.966588) (width 0.25) (layer "F.Cu") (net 3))
 (segment (start 25.491322 53.574501) (end 27.421175 53.574501) (width 0.25) (layer "F.Cu") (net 3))
 (segment (start 32.733412 52.966588) (end 32.75 52.95) (width 0.25) (layer "F.Cu") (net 3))
 (segment (start 24.883409 52.966588) (end 25.491322 53.574501) (width 0.25) (layer "F.Cu") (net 3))
 (segment (start 20.479088 52.966588) (end 24.883409 52.966588) (width 0.25) (layer "F.Cu") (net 3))
 (segment (start 28.029088 52.966588) (end 32.733412 52.966588) (width 0.25) (layer "F.Cu") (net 3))
 (via (at 32.75 52.95) (size 0.7) (drill 0.4) (layers "F.Cu" "B.Cu") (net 3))
 (segment (start 32 53.105) (end 32.595 53.105) (width 0.25) (layer "B.Cu") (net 3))
 (segment (start 32.595 53.105) (end 32.75 52.95) (width 0.25) (layer "B.Cu") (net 3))
 (segment (start 21.2125 51.2) (end 27.295676 51.2) (width 0.25) (layer "F.Cu") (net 2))
 (segment (start 20.7125 50.7) (end 21.2125 51.2) (width 0.25) (layer "F.Cu") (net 2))
 (segment (start 29.668172 52.265105) (end 29.668172 52.105672) (width 0.25) (layer "F.Cu") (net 2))
 (segment (start 29.668172 52.105672) (end 28.029088 50.466588) (width 0.25) (layer "F.Cu") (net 2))
 (segment (start 27.295676 51.2) (end 27.795676 50.7) (width 0.25) (layer "F.Cu") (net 2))
 (via (at 29.668172 52.265105) (size 0.7) (drill 0.4) (layers "F.Cu" "B.Cu") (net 2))
 (segment (start 30.73 54.375) (end 30.162923 54.942077) (width 0.25) (layer "B.Cu") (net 2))
 (segment (start 30.162923 54.942077) (end 29.10049 54.942077) (width 0.25) (layer "B.Cu") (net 2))
 (segment (start 29.10049 52.832787) (end 29.668172 52.265105) (width 0.25) (layer "B.Cu") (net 2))
 (segment (start 29.10049 54.942077) (end 29.10049 52.832787) (width 0.25) (layer "B.Cu") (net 2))
 (segment (start 28.029088 55.466588) (end 29.381098 54.114578) (width 0.25) (layer "F.Cu") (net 4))
 (segment (start 25.25 56.2) (end 27.295676 56.2) (width 0.25) (layer "F.Cu") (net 4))
 (segment (start 20.479088 55.466588) (end 24.516588 55.466588) (width 0.25) (layer "F.Cu") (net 4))
 (segment (start 24.516588 55.466588) (end 25.25 56.2) (width 0.25) (layer "F.Cu") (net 4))
 (segment (start 27.295676 56.2) (end 28.029088 55.466588) (width 0.25) (layer "F.Cu") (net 4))
 (segment (start 29.381098 54.114578) (end 29.758188 54.114578) (width 0.25) (layer "F.Cu") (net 4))
 (via (at 29.758188 54.114578) (size 0.7) (drill 0.4) (layers "F.Cu" "B.Cu") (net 4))
 (segment (start 30.73 53.105) (end 29.758188 54.076812) (width 0.25) (layer "B.Cu") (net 4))
 (segment (start 29.758188 54.076812) (end 29.758188 54.114578) (width 0.25) (layer "B.Cu") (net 4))
 (segment (start 27.0125 54.7) (end 27.779088 55.466588) (width 0.5) (layer "B.Cu") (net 5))
 (segment (start 23.75 55.45) (end 24.5 54.7) (width 0.5) (layer "B.Cu") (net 5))
 (segment (start 32.9 50.565) (end 33.768137 51.433137) (width 0.5) (layer "B.Cu") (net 5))
 (segment (start 24.5 54.7) (end 27.0125 54.7) (width 0.5) (layer "B.Cu") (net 5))
 (segment (start 32.867913 55.466588) (end 27.779088 55.466588) (width 0.5) (layer "B.Cu") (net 5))
 (segment (start 32 50.565) (end 32.9 50.565) (width 0.5) (layer "B.Cu") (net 5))
 (segment (start 20.529088 55.466588) (end 20.545676 55.45) (width 0.5) (layer "B.Cu") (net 5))
 (segment (start 33.768137 51.433137) (end 33.768137 54.566364) (width 0.5) (layer "B.Cu") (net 5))
 (segment (start 20.545676 55.45) (end 23.75 55.45) (width 0.5) (layer "B.Cu") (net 5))
 (segment (start 33.768137 54.566364) (end 32.867913 55.466588) (width 0.5) (layer "B.Cu") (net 5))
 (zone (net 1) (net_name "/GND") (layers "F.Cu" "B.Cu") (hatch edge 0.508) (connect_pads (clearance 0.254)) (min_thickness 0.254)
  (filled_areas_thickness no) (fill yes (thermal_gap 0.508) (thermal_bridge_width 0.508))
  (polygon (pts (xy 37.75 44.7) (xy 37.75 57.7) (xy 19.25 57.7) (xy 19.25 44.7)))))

